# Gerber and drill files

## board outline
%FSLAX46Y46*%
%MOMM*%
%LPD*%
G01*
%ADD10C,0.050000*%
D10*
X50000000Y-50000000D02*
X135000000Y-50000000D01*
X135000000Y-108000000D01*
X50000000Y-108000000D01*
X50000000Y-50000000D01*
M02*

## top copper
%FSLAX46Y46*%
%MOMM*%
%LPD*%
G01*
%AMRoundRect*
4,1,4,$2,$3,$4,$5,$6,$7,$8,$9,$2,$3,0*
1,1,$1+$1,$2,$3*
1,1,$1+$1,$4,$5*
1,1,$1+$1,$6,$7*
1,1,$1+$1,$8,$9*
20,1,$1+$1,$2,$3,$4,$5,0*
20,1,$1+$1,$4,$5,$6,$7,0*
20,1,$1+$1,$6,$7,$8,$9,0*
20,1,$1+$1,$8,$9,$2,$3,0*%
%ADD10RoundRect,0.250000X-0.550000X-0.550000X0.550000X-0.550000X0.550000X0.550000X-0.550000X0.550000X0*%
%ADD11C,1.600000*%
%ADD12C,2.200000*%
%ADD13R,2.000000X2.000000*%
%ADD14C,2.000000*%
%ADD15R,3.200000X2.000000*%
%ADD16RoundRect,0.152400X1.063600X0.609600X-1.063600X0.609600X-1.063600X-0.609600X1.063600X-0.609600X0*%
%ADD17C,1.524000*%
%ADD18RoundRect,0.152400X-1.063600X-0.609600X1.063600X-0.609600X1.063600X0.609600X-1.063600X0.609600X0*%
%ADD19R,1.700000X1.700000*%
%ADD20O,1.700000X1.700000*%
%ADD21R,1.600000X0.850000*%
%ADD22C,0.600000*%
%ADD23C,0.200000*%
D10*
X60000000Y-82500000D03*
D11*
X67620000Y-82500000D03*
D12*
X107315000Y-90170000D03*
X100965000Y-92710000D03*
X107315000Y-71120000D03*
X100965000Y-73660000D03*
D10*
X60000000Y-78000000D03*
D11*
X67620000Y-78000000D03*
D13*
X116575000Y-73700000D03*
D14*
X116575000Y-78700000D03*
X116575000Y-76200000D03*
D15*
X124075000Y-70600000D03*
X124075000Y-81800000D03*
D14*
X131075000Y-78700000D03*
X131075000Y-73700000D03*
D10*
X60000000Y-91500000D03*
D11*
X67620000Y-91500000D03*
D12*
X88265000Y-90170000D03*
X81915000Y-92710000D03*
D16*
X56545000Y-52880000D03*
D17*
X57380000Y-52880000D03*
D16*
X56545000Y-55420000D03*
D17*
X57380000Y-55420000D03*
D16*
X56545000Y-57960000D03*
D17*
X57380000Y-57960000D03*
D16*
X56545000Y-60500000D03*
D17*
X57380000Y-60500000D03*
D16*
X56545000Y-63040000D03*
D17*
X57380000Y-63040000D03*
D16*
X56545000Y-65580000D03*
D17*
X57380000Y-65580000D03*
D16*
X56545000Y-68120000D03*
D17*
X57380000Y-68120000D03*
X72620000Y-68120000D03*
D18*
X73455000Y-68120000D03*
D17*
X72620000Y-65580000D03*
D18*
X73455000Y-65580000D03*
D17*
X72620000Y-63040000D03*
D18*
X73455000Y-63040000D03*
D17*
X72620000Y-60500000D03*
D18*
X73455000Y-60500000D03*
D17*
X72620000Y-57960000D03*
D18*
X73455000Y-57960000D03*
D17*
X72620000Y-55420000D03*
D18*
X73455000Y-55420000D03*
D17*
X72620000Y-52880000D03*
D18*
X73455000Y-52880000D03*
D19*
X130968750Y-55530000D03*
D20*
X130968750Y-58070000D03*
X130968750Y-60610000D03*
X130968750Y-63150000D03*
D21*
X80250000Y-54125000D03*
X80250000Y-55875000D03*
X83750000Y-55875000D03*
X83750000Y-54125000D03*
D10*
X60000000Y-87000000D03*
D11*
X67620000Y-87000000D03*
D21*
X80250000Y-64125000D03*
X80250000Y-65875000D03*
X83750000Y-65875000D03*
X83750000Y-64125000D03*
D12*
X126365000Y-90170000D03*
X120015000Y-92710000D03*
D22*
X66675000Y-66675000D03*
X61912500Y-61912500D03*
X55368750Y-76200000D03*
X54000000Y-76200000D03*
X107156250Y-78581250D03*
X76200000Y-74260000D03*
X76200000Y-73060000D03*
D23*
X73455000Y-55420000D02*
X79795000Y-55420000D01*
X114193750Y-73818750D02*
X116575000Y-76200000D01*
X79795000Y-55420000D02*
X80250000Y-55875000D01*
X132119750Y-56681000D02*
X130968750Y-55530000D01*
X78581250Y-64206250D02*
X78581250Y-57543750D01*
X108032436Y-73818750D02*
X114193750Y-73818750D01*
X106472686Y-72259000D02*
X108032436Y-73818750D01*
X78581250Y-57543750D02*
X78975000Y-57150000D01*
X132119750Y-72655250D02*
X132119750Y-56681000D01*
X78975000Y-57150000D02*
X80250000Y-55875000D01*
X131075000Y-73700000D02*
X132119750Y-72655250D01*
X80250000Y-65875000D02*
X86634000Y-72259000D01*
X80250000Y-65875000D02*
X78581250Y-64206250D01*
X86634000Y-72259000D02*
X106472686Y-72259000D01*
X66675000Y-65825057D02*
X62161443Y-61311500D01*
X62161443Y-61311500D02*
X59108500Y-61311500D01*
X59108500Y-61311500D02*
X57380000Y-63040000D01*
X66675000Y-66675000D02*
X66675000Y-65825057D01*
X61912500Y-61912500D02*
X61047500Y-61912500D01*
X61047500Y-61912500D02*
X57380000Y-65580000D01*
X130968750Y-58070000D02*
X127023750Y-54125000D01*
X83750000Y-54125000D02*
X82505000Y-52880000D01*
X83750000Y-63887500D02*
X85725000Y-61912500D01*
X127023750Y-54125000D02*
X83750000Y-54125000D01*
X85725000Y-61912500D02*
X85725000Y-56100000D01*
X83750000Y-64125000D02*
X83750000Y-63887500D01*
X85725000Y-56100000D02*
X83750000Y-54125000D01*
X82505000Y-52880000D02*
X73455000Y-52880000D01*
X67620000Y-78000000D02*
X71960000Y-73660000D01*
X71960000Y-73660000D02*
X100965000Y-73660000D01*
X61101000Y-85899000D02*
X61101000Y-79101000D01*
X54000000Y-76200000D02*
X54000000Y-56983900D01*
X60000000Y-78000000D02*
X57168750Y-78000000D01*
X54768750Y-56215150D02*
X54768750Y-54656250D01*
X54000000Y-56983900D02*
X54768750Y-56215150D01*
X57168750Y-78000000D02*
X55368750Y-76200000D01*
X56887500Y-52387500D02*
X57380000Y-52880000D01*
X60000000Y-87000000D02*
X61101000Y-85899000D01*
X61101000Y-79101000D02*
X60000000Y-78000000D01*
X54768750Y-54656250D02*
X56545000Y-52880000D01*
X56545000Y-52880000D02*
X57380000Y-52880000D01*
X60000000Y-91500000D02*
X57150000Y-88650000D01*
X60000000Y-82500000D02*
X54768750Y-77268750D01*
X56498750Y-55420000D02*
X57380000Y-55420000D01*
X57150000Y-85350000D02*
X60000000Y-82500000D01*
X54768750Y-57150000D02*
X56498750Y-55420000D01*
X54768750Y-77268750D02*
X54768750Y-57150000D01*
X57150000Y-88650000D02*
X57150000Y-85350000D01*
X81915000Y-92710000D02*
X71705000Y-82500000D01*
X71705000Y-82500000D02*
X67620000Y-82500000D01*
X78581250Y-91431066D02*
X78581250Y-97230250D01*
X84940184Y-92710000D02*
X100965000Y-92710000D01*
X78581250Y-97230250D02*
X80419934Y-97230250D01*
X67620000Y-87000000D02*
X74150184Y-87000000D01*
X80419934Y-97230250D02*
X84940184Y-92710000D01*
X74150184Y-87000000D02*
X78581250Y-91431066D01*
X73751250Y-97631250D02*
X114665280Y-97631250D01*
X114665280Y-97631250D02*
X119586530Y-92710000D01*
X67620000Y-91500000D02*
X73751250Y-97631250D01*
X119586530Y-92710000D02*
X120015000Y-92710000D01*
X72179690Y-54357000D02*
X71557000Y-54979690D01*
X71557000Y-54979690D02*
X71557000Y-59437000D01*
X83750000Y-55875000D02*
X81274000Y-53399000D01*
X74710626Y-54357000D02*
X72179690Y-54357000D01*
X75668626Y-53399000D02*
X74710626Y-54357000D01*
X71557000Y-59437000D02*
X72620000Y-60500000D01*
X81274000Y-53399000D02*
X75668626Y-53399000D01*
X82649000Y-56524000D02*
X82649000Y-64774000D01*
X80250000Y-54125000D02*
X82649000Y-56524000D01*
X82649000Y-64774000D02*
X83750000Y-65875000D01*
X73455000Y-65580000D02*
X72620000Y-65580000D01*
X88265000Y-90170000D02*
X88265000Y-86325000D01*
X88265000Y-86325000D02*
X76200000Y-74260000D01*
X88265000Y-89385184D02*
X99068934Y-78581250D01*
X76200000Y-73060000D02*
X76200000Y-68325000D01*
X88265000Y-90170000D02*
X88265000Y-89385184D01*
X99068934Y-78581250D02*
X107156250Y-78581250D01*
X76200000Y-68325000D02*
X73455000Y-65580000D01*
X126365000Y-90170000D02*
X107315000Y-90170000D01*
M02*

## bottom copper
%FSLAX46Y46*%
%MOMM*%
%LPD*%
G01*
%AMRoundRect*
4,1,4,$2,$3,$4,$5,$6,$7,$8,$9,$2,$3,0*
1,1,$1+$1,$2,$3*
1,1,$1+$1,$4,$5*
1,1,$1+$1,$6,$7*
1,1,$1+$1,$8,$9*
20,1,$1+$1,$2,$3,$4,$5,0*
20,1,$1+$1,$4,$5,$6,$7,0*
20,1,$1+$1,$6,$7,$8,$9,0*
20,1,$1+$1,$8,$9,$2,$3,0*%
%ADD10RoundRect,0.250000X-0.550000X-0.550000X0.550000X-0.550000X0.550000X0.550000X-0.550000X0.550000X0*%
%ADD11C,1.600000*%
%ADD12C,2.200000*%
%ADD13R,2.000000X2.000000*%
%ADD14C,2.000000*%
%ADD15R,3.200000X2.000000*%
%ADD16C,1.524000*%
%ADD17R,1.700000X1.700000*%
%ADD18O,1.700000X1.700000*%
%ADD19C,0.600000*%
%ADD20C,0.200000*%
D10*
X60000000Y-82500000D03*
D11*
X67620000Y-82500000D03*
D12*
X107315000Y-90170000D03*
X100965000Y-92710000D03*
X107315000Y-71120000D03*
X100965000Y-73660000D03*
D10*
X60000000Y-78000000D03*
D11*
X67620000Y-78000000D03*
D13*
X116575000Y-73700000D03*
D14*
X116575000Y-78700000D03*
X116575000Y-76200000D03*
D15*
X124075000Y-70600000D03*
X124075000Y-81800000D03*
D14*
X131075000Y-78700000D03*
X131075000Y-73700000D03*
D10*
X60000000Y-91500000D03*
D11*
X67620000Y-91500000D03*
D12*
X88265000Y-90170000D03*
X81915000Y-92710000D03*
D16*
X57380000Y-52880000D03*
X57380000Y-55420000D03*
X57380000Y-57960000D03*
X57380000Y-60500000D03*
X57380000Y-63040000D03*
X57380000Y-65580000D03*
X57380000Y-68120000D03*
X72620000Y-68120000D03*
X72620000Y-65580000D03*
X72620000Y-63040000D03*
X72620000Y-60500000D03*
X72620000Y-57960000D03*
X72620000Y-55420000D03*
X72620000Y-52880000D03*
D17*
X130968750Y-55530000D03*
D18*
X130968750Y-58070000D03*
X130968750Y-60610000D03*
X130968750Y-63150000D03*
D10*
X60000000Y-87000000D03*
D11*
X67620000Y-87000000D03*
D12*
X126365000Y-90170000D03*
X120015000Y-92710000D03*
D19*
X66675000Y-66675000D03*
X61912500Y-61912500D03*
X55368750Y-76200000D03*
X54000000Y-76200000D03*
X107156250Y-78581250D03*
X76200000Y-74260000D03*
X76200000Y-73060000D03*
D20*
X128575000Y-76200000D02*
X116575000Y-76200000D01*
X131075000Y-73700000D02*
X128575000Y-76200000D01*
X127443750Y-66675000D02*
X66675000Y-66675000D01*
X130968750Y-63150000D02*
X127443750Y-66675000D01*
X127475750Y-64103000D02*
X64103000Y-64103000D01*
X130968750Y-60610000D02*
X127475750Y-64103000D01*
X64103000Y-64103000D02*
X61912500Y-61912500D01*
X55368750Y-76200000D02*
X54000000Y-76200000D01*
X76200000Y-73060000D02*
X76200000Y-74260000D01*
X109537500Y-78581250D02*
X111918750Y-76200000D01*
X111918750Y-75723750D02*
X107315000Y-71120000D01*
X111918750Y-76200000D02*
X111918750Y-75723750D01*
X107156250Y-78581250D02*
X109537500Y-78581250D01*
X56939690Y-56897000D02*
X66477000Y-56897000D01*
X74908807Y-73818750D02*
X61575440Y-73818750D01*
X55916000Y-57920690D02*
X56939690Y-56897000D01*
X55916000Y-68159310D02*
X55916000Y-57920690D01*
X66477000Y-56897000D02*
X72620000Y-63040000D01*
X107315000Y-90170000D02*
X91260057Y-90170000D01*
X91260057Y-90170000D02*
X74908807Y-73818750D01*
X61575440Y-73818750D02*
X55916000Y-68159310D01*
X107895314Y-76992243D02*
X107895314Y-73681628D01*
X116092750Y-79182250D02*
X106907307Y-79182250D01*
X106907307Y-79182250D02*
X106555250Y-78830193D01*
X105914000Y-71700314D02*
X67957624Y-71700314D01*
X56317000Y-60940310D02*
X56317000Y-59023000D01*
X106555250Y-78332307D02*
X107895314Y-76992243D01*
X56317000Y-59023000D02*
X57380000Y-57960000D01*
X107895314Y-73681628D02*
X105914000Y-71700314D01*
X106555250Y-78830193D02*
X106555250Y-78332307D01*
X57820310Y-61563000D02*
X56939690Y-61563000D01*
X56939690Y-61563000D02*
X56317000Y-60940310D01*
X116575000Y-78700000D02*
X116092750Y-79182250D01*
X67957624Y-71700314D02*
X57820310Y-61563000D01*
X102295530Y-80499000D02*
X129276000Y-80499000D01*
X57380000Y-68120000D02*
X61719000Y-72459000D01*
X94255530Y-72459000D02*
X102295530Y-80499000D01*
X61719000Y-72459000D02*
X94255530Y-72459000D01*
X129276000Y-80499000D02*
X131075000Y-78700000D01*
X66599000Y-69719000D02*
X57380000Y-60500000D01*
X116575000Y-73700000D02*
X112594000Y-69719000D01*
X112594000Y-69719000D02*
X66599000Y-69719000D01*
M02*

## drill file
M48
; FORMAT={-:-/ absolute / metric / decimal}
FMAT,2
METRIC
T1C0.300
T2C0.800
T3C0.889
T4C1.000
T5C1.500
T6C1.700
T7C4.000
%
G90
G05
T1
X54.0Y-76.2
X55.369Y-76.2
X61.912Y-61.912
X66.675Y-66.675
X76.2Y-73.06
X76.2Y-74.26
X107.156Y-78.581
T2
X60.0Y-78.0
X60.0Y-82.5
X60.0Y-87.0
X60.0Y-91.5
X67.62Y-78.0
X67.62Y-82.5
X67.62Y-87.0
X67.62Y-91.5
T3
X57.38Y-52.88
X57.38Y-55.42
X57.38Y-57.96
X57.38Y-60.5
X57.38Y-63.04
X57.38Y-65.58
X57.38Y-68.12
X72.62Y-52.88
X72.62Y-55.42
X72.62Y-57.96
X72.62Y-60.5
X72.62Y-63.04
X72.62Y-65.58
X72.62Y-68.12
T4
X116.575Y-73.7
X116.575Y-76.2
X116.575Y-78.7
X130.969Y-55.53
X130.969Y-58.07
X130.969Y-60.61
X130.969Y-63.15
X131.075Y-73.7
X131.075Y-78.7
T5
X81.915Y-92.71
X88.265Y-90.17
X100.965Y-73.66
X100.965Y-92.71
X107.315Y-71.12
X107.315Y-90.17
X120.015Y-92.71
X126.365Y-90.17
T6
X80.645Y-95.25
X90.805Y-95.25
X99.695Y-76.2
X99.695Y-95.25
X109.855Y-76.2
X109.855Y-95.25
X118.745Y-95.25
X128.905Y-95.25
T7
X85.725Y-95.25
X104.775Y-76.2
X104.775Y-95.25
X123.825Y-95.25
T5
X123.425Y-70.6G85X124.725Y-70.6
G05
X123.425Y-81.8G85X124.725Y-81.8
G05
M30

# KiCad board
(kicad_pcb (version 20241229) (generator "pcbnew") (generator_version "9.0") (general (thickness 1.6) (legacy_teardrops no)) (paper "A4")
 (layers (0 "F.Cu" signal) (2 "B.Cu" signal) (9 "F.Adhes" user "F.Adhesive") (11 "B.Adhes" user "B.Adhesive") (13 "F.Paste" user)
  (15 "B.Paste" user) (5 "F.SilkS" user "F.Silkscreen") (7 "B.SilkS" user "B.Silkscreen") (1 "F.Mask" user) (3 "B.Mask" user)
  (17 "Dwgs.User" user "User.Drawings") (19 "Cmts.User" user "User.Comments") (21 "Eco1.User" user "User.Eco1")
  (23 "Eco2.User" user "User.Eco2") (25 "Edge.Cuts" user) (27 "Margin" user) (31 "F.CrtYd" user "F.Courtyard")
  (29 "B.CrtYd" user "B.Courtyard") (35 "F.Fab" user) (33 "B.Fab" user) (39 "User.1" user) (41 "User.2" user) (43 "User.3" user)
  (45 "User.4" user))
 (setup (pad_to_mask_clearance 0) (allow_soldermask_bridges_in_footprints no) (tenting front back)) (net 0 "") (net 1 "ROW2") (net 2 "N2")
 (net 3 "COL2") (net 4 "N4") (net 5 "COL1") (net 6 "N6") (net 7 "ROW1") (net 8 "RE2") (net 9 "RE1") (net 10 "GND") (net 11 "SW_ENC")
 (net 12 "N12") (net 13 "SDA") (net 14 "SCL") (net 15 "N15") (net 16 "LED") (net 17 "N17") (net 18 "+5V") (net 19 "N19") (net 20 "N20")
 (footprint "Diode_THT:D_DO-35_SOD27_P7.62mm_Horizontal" (layer "F.Cu") (at 60 82.5)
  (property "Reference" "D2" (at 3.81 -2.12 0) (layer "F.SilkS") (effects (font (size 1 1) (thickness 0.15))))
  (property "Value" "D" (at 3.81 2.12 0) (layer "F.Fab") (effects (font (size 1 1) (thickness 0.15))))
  (pad "1" thru_hole roundrect (at 0 0) (size 1.6 1.6) (drill 0.8) (layers "*.Cu" "*.Mask") (remove_unused_layers no)
   (roundrect_rratio 0.15625) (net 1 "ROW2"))
  (pad "2" thru_hole circle (at 7.62 0) (size 1.6 1.6) (drill 0.8) (layers "*.Cu" "*.Mask") (remove_unused_layers no) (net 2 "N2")))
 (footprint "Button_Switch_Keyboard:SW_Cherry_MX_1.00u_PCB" (layer "F.Cu") (at 107.315 90.17)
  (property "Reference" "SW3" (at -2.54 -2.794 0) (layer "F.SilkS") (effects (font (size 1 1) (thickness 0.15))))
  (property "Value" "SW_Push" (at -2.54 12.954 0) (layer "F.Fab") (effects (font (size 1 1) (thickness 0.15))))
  (pad "" np_thru_hole circle (at -7.62 5.08) (size 1.7 1.7) (drill 1.7) (layers "*.Cu" "*.Mask"))
  (pad "" np_thru_hole circle (at -2.54 5.08) (size 4 4) (drill 4) (layers "*.Cu" "*.Mask"))
  (pad "" np_thru_hole circle (at 2.54 5.08) (size 1.7 1.7) (drill 1.7) (layers "*.Cu" "*.Mask"))
  (pad "1" thru_hole circle (at 0 0) (size 2.2 2.2) (drill 1.5) (layers "*.Cu" "*.Mask") (remove_unused_layers no) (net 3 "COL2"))
  (pad "2" thru_hole circle (at -6.35 2.54) (size 2.2 2.2) (drill 1.5) (layers "*.Cu" "*.Mask") (remove_unused_layers no) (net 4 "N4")))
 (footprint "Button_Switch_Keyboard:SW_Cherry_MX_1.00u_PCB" (layer "F.Cu") (at 107.315 71.12)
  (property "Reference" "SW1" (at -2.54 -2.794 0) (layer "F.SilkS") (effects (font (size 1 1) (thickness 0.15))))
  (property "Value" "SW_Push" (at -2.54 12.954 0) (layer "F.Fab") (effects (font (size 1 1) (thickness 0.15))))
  (pad "" np_thru_hole circle (at -7.62 5.08) (size 1.7 1.7) (drill 1.7) (layers "*.Cu" "*.Mask"))
  (pad "" np_thru_hole circle (at -2.54 5.08) (size 4 4) (drill 4) (layers "*.Cu" "*.Mask"))
  (pad "" np_thru_hole circle (at 2.54 5.08) (size 1.7 1.7) (drill 1.7) (layers "*.Cu" "*.Mask"))
  (pad "1" thru_hole circle (at 0 0) (size 2.2 2.2) (drill 1.5) (layers "*.Cu" "*.Mask") (remove_unused_layers no) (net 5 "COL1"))
  (pad "2" thru_hole circle (at -6.35 2.54) (size 2.2 2.2) (drill 1.5) (layers "*.Cu" "*.Mask") (remove_unused_layers no) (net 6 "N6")))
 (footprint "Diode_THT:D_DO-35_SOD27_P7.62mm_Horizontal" (layer "F.Cu") (at 60 78)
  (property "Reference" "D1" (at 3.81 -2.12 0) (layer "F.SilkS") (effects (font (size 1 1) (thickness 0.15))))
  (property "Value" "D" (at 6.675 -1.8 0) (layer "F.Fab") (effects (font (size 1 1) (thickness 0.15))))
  (pad "1" thru_hole roundrect (at 0 0) (size 1.6 1.6) (drill 0.8) (layers "*.Cu" "*.Mask") (remove_unused_layers no)
   (roundrect_rratio 0.15625) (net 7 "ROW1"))
  (pad "2" thru_hole circle (at 7.62 0) (size 1.6 1.6) (drill 0.8) (layers "*.Cu" "*.Mask") (remove_unused_layers no) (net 6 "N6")))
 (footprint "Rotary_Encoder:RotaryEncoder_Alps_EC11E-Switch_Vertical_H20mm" (layer "F.Cu") (at 116.575 73.7)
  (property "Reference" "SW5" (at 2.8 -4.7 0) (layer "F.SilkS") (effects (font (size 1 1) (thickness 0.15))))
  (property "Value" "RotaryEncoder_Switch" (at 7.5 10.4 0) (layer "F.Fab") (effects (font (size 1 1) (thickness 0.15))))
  (pad "A" thru_hole rect (at 0 0) (size 2 2) (drill 1) (layers "*.Cu" "*.Mask") (remove_unused_layers no) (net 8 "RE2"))
  (pad "B" thru_hole circle (at 0 5) (size 2 2) (drill 1) (layers "*.Cu" "*.Mask") (remove_unused_layers no) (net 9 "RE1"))
  (pad "C" thru_hole circle (at 0 2.5) (size 2 2) (drill 1) (layers "*.Cu" "*.Mask") (remove_unused_layers no) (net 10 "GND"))
  (pad "MP" thru_hole rect (at 7.5 -3.1) (size 3.2 2) (drill oval 2.8 1.5) (layers "*.Cu" "*.Mask") (remove_unused_layers no))
  (pad "MP" thru_hole rect (at 7.5 8.1) (size 3.2 2) (drill oval 2.8 1.5) (layers "*.Cu" "*.Mask") (remove_unused_layers no))
  (pad "S1" thru_hole circle (at 14.5 5) (size 2 2) (drill 1) (layers "*.Cu" "*.Mask") (remove_unused_layers no) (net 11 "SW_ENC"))
  (pad "S2" thru_hole circle (at 14.5 0) (size 2 2) (drill 1) (layers "*.Cu" "*.Mask") (remove_unused_layers no) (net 10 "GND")))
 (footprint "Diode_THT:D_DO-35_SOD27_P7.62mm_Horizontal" (layer "F.Cu") (at 60 91.5)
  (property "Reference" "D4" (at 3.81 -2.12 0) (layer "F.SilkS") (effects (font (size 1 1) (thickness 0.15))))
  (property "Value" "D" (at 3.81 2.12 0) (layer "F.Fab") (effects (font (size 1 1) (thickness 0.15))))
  (pad "1" thru_hole roundrect (at 0 0) (size 1.6 1.6) (drill 0.8) (layers "*.Cu" "*.Mask") (remove_unused_layers no)
   (roundrect_rratio 0.15625) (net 1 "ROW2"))
  (pad "2" thru_hole circle (at 7.62 0) (size 1.6 1.6) (drill 0.8) (layers "*.Cu" "*.Mask") (remove_unused_layers no) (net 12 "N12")))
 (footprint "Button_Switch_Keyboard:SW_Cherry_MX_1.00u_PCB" (layer "F.Cu") (at 88.265 90.17)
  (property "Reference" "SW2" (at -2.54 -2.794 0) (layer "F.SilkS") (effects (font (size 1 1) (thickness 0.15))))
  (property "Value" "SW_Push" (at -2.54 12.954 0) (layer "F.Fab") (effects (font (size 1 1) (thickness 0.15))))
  (pad "" np_thru_hole circle (at -7.62 5.08) (size 1.7 1.7) (drill 1.7) (layers "*.Cu" "*.Mask"))
  (pad "" np_thru_hole circle (at -2.54 5.08) (size 4 4) (drill 4) (layers "*.Cu" "*.Mask"))
  (pad "" np_thru_hole circle (at 2.54 5.08) (size 1.7 1.7) (drill 1.7) (layers "*.Cu" "*.Mask"))
  (pad "1" thru_hole circle (at 0 0) (size 2.2 2.2) (drill 1.5) (layers "*.Cu" "*.Mask") (remove_unused_layers no) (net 5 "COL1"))
  (pad "2" thru_hole circle (at -6.35 2.54) (size 2.2 2.2) (drill 1.5) (layers "*.Cu" "*.Mask") (remove_unused_layers no) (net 2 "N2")))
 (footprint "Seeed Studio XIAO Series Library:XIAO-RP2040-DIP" (layer "F.Cu") (at 65 60.5)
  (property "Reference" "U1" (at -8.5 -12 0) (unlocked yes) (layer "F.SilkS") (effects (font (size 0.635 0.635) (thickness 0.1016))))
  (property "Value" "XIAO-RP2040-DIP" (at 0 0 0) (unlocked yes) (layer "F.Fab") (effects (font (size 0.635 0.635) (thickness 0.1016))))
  (pad "1" smd roundrect (at -8.455 -7.62 180) (size 2.432 1.524) (layers "F.Cu" "F.Mask") (roundrect_rratio 0.1) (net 7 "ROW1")
   (thermal_bridge_angle 45))
  (pad "1" thru_hole circle (at -7.62 -7.62 180) (size 1.524 1.524) (drill 0.889) (layers "*.Cu" "*.Mask") (remove_unused_layers no)
   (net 7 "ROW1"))
  (pad "2" smd roundrect (at -8.455 -5.08 180) (size 2.432 1.524) (layers "F.Cu" "F.Mask") (roundrect_rratio 0.1) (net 1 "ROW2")
   (thermal_bridge_angle 45))
  (pad "2" thru_hole circle (at -7.62 -5.08 180) (size 1.524 1.524) (drill 0.889) (layers "*.Cu" "*.Mask") (remove_unused_layers no)
   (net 1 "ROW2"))
  (pad "3" smd roundrect (at -8.455 -2.54 180) (size 2.432 1.524) (layers "F.Cu" "F.Mask") (roundrect_rratio 0.1) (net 9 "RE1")
   (thermal_bridge_angle 45))
  (pad "3" thru_hole circle (at -7.62 -2.54 180) (size 1.524 1.524) (drill 0.889) (layers "*.Cu" "*.Mask") (remove_unused_layers no)
   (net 9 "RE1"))
  (pad "4" smd roundrect (at -8.455 0 180) (size 2.432 1.524) (layers "F.Cu" "F.Mask") (roundrect_rratio 0.1) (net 8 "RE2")
   (thermal_bridge_angle 45))
  (pad "4" thru_hole circle (at -7.62 0 180) (size 1.524 1.524) (drill 0.889) (layers "*.Cu" "*.Mask") (remove_unused_layers no)
   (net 8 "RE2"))
  (pad "5" smd roundrect (at -8.455 2.54 180) (size 2.432 1.524) (layers "F.Cu" "F.Mask") (roundrect_rratio 0.1) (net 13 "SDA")
   (thermal_bridge_angle 45))
  (pad "5" thru_hole circle (at -7.62 2.54 180) (size 1.524 1.524) (drill 0.889) (layers "*.Cu" "*.Mask") (remove_unused_layers no)
   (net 13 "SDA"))
  (pad "6" smd roundrect (at -8.455 5.08 180) (size 2.432 1.524) (layers "F.Cu" "F.Mask") (roundrect_rratio 0.1) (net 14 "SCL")
   (thermal_bridge_angle 45))
  (pad "6" thru_hole circle (at -7.62 5.08 180) (size 1.524 1.524) (drill 0.889) (layers "*.Cu" "*.Mask") (remove_unused_layers no)
   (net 14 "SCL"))
  (pad "7" smd roundrect (at -8.455 7.62 180) (size 2.432 1.524) (layers "F.Cu" "F.Mask") (roundrect_rratio 0.1) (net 11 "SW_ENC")
   (thermal_bridge_angle 45))
  (pad "7" thru_hole circle (at -7.62 7.62 180) (size 1.524 1.524) (drill 0.889) (layers "*.Cu" "*.Mask") (remove_unused_layers no)
   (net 11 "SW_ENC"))
  (pad "8" thru_hole circle (at 7.62 7.62) (size 1.524 1.524) (drill 0.889) (layers "*.Cu" "*.Mask") (remove_unused_layers no)
   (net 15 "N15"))
  (pad "8" smd roundrect (at 8.455 7.62) (size 2.432 1.524) (layers "F.Cu" "F.Mask") (roundrect_rratio 0.1) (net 15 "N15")
   (thermal_bridge_angle 45))
  (pad "9" thru_hole circle (at 7.62 5.08) (size 1.524 1.524) (drill 0.889) (layers "*.Cu" "*.Mask") (remove_unused_layers no)
   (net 5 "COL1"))
  (pad "9" smd roundrect (at 8.455 5.08) (size 2.432 1.524) (layers "F.Cu" "F.Mask") (roundrect_rratio 0.1) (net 5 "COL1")
   (thermal_bridge_angle 45))
  (pad "10" thru_hole circle (at 7.62 2.54) (size 1.524 1.524) (drill 0.889) (layers "*.Cu" "*.Mask") (remove_unused_layers no)
   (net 3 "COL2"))
  (pad "10" smd roundrect (at 8.455 2.54) (size 2.432 1.524) (layers "F.Cu" "F.Mask") (roundrect_rratio 0.1) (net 3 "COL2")
   (thermal_bridge_angle 45))
  (pad "11" thru_hole circle (at 7.62 0) (size 1.524 1.524) (drill 0.889) (layers "*.Cu" "*.Mask") (remove_unused_layers no) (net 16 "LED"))
  (pad "11" smd roundrect (at 8.455 0) (size 2.432 1.524) (layers "F.Cu" "F.Mask") (roundrect_rratio 0.1) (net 16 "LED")
   (thermal_bridge_angle 45))
  (pad "12" thru_hole circle (at 7.62 -2.54) (size 1.524 1.524) (drill 0.889) (layers "*.Cu" "*.Mask") (remove_unused_layers no)
   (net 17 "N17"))
  (pad "12" smd roundrect (at 8.455 -2.54) (size 2.432 1.524) (layers "F.Cu" "F.Mask") (roundrect_rratio 0.1) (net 17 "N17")
   (thermal_bridge_angle 45))
  (pad "13" thru_hole circle (at 7.62 -5.08) (size 1.524 1.524) (drill 0.889) (layers "*.Cu" "*.Mask") (remove_unused_layers no)
   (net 10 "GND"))
  (pad "13" smd roundrect (at 8.455 -5.08) (size 2.432 1.524) (layers "F.Cu" "F.Mask") (roundrect_rratio 0.1) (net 10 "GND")
   (thermal_bridge_angle 45))
  (pad "14" thru_hole circle (at 7.62 -7.62) (size 1.524 1.524) (drill 0.889) (layers "*.Cu" "*.Mask") (remove_unused_layers no)
   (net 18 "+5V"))
  (pad "14" smd roundrect (at 8.455 -7.62) (size 2.432 1.524) (layers "F.Cu" "F.Mask") (roundrect_rratio 0.1) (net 18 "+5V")
   (thermal_bridge_angle 45)))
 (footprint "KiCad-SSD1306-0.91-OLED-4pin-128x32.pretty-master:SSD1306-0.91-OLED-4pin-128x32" (layer "F.Cu") (at 94.46875 53.34)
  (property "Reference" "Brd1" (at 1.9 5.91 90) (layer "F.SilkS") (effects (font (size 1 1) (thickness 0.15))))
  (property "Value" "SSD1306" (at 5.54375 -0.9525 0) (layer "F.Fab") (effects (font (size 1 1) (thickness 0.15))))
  (pad "1" thru_hole rect (at 36.5 2.19) (size 1.7 1.7) (drill 1) (layers "*.Cu" "*.Mask") (remove_unused_layers no) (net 10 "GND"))
  (pad "2" thru_hole oval (at 36.5 4.73) (size 1.7 1.7) (drill 1) (layers "*.Cu" "*.Mask") (remove_unused_layers no) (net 18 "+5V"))
  (pad "3" thru_hole oval (at 36.5 7.27) (size 1.7 1.7) (drill 1) (layers "*.Cu" "*.Mask") (remove_unused_layers no) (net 14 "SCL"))
  (pad "4" thru_hole oval (at 36.5 9.81) (size 1.7 1.7) (drill 1) (layers "*.Cu" "*.Mask") (remove_unused_layers no) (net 13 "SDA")))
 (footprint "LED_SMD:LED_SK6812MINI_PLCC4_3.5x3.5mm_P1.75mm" (layer "F.Cu") (at 82 55)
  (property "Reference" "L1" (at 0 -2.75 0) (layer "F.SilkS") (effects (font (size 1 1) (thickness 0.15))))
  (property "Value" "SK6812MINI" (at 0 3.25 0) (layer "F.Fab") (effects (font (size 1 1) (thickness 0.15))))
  (pad "1" smd rect (at -1.75 -0.875) (size 1.6 0.85) (layers "F.Cu" "F.Mask" "F.Paste") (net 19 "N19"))
  (pad "2" smd rect (at -1.75 0.875) (size 1.6 0.85) (layers "F.Cu" "F.Mask" "F.Paste") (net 10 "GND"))
  (pad "3" smd rect (at 1.75 0.875) (size 1.6 0.85) (layers "F.Cu" "F.Mask" "F.Paste") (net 16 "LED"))
  (pad "4" smd rect (at 1.75 -0.875) (size 1.6 0.85) (layers "F.Cu" "F.Mask" "F.Paste") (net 18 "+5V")))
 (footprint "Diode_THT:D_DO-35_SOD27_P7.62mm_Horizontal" (layer "F.Cu") (at 60 87)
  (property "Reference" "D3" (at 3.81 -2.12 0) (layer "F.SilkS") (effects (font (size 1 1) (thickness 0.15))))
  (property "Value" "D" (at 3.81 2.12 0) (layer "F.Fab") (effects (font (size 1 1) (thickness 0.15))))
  (pad "1" thru_hole roundrect (at 0 0) (size 1.6 1.6) (drill 0.8) (layers "*.Cu" "*.Mask") (remove_unused_layers no)
   (roundrect_rratio 0.15625) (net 7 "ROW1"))
  (pad "2" thru_hole circle (at 7.62 0) (size 1.6 1.6) (drill 0.8) (layers "*.Cu" "*.Mask") (remove_unused_layers no) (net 4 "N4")))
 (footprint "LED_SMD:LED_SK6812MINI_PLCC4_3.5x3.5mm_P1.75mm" (layer "F.Cu") (at 82 65)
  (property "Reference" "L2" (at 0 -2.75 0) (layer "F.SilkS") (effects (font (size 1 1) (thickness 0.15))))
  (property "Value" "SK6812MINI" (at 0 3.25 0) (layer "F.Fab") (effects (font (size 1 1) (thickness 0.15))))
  (pad "1" smd rect (at -1.75 -0.875) (size 1.6 0.85) (layers "F.Cu" "F.Mask" "F.Paste") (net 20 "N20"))
  (pad "2" smd rect (at -1.75 0.875) (size 1.6 0.85) (layers "F.Cu" "F.Mask" "F.Paste") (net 10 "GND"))
  (pad "3" smd rect (at 1.75 0.875) (size 1.6 0.85) (layers "F.Cu" "F.Mask" "F.Paste") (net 19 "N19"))
  (pad "4" smd rect (at 1.75 -0.875) (size 1.6 0.85) (layers "F.Cu" "F.Mask" "F.Paste") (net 18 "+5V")))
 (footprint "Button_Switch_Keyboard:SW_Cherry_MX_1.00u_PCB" (layer "F.Cu") (at 126.365 90.17)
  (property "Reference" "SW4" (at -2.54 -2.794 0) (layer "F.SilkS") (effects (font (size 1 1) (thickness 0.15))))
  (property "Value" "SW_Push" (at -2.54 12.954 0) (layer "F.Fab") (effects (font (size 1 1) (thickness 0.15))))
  (pad "" np_thru_hole circle (at -7.62 5.08) (size 1.7 1.7) (drill 1.7) (layers "*.Cu" "*.Mask"))
  (pad "" np_thru_hole circle (at -2.54 5.08) (size 4 4) (drill 4) (layers "*.Cu" "*.Mask"))
  (pad "" np_thru_hole circle (at 2.54 5.08) (size 1.7 1.7) (drill 1.7) (layers "*.Cu" "*.Mask"))
  (pad "1" thru_hole circle (at 0 0) (size 2.2 2.2) (drill 1.5) (layers "*.Cu" "*.Mask") (remove_unused_layers no) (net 3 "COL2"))
  (pad "2" thru_hole circle (at -6.35 2.54) (size 2.2 2.2) (drill 1.5) (layers "*.Cu" "*.Mask") (remove_unused_layers no) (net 12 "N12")))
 (gr_rect (start 50 50) (end 135 108) (stroke (width 0.05) (type solid)) (fill no) (layer "Edge.Cuts"))
 (segment (start 73.455 55.42) (end 79.795 55.42) (width 0.2) (layer "F.Cu") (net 10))
 (segment (start 114.19375 73.81875) (end 116.575 76.2) (width 0.2) (layer "F.Cu") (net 10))
 (segment (start 79.795 55.42) (end 80.25 55.875) (width 0.2) (layer "F.Cu") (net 10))
 (segment (start 132.11975 56.681) (end 130.96875 55.53) (width 0.2) (layer "F.Cu") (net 10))
 (segment (start 78.58125 64.20625) (end 78.58125 57.54375) (width 0.2) (layer "F.Cu") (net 10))
 (segment (start 108.032436 73.81875) (end 114.19375 73.81875) (width 0.2) (layer "F.Cu") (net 10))
 (segment (start 106.472686 72.259) (end 108.032436 73.81875) (width 0.2) (layer "F.Cu") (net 10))
 (segment (start 78.58125 57.54375) (end 78.975 57.15) (width 0.2) (layer "F.Cu") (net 10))
 (segment (start 132.11975 72.65525) (end 132.11975 56.681) (width 0.2) (layer "F.Cu") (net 10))
 (segment (start 78.975 57.15) (end 80.25 55.875) (width 0.2) (layer "F.Cu") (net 10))
 (segment (start 131.075 73.7) (end 132.11975 72.65525) (width 0.2) (layer "F.Cu") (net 10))
 (segment (start 80.25 65.875) (end 86.634 72.259) (width 0.2) (layer "F.Cu") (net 10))
 (segment (start 80.25 65.875) (end 78.58125 64.20625) (width 0.2) (layer "F.Cu") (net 10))
 (segment (start 86.634 72.259) (end 106.472686 72.259) (width 0.2) (layer "F.Cu") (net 10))
 (segment (start 128.575 76.2) (end 116.575 76.2) (width 0.2) (layer "B.Cu") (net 10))
 (segment (start 131.075 73.7) (end 128.575 76.2) (width 0.2) (layer "B.Cu") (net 10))
 (segment (start 66.675 65.825057) (end 62.161443 61.3115) (width 0.2) (layer "F.Cu") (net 13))
 (segment (start 62.161443 61.3115) (end 59.1085 61.3115) (width 0.2) (layer "F.Cu") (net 13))
 (segment (start 59.1085 61.3115) (end 57.38 63.04) (width 0.2) (layer "F.Cu") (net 13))
 (segment (start 66.675 66.675) (end 66.675 65.825057) (width 0.2) (layer "F.Cu") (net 13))
 (via (at 66.675 66.675) (size 0.6) (drill 0.3) (layers "F.Cu" "B.Cu") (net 13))
 (segment (start 127.44375 66.675) (end 66.675 66.675) (width 0.2) (layer "B.Cu") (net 13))
 (segment (start 130.96875 63.15) (end 127.44375 66.675) (width 0.2) (layer "B.Cu") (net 13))
 (segment (start 61.9125 61.9125) (end 61.0475 61.9125) (width 0.2) (layer "F.Cu") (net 14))
 (segment (start 61.0475 61.9125) (end 57.38 65.58) (width 0.2) (layer "F.Cu") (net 14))
 (via (at 61.9125 61.9125) (size 0.6) (drill 0.3) (layers "F.Cu" "B.Cu") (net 14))
 (segment (start 127.47575 64.103) (end 64.103 64.103) (width 0.2) (layer "B.Cu") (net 14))
 (segment (start 130.96875 60.61) (end 127.47575 64.103) (width 0.2) (layer "B.Cu") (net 14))
 (segment (start 64.103 64.103) (end 61.9125 61.9125) (width 0.2) (layer "B.Cu") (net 14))
 (segment (start 130.96875 58.07) (end 127.02375 54.125) (width 0.2) (layer "F.Cu") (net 18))
 (segment (start 83.75 54.125) (end 82.505 52.88) (width 0.2) (layer "F.Cu") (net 18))
 (segment (start 83.75 63.8875) (end 85.725 61.9125) (width 0.2) (layer "F.Cu") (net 18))
 (segment (start 127.02375 54.125) (end 83.75 54.125) (width 0.2) (layer "F.Cu") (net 18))
 (segment (start 85.725 61.9125) (end 85.725 56.1) (width 0.2) (layer "F.Cu") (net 18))
 (segment (start 83.75 64.125) (end 83.75 63.8875) (width 0.2) (layer "F.Cu") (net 18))
 (segment (start 85.725 56.1) (end 83.75 54.125) (width 0.2) (layer "F.Cu") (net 18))
 (segment (start 82.505 52.88) (end 73.455 52.88) (width 0.2) (layer "F.Cu") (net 18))
 (segment (start 67.62 78) (end 71.96 73.66) (width 0.2) (layer "F.Cu") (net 6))
 (segment (start 71.96 73.66) (end 100.965 73.66) (width 0.2) (layer "F.Cu") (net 6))
 (segment (start 61.101 85.899) (end 61.101 79.101) (width 0.2) (layer "F.Cu") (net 7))
 (segment (start 54 76.2) (end 54 56.9839) (width 0.2) (layer "F.Cu") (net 7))
 (segment (start 60 78) (end 57.16875 78) (width 0.2) (layer "F.Cu") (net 7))
 (segment (start 54.76875 56.21515) (end 54.76875 54.65625) (width 0.2) (layer "F.Cu") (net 7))
 (segment (start 54 56.9839) (end 54.76875 56.21515) (width 0.2) (layer "F.Cu") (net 7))
 (segment (start 57.16875 78) (end 55.36875 76.2) (width 0.2) (layer "F.Cu") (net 7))
 (segment (start 56.8875 52.3875) (end 57.38 52.88) (width 0.2) (layer "F.Cu") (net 7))
 (segment (start 60 87) (end 61.101 85.899) (width 0.2) (layer "F.Cu") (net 7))
 (segment (start 61.101 79.101) (end 60 78) (width 0.2) (layer "F.Cu") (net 7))
 (segment (start 54.76875 54.65625) (end 56.545 52.88) (width 0.2) (layer "F.Cu") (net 7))
 (segment (start 56.545 52.88) (end 57.38 52.88) (width 0.2) (layer "F.Cu") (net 7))
 (via (at 55.36875 76.2) (size 0.6) (drill 0.3) (layers "F.Cu" "B.Cu") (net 7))
 (via (at 54 76.2) (size 0.6) (drill 0.3) (layers "F.Cu" "B.Cu") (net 7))
 (segment (start 55.36875 76.2) (end 54 76.2) (width 0.2) (layer "B.Cu") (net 7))
 (segment (start 60 91.5) (end 57.15 88.65) (width 0.2) (layer "F.Cu") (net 1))
 (segment (start 60 82.5) (end 54.76875 77.26875) (width 0.2) (layer "F.Cu") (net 1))
 (segment (start 56.49875 55.42) (end 57.38 55.42) (width 0.2) (layer "F.Cu") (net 1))
 (segment (start 57.15 85.35) (end 60 82.5) (width 0.2) (layer "F.Cu") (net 1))
 (segment (start 54.76875 57.15) (end 56.49875 55.42) (width 0.2) (layer "F.Cu") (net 1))
 (segment (start 54.76875 77.26875) (end 54.76875 57.15) (width 0.2) (layer "F.Cu") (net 1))
 (segment (start 57.15 88.65) (end 57.15 85.35) (width 0.2) (layer "F.Cu") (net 1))
 (segment (start 81.915 92.71) (end 71.705 82.5) (width 0.2) (layer "F.Cu") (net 2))
 (segment (start 71.705 82.5) (end 67.62 82.5) (width 0.2) (layer "F.Cu") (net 2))
 (segment (start 78.58125 91.431066) (end 78.58125 97.23025) (width 0.2) (layer "F.Cu") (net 4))
 (segment (start 84.940184 92.71) (end 100.965 92.71) (width 0.2) (layer "F.Cu") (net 4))
 (segment (start 78.58125 97.23025) (end 80.419934 97.23025) (width 0.2) (layer "F.Cu") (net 4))
 (segment (start 67.62 87) (end 74.150184 87) (width 0.2) (layer "F.Cu") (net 4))
 (segment (start 80.419934 97.23025) (end 84.940184 92.71) (width 0.2) (layer "F.Cu") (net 4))
 (segment (start 74.150184 87) (end 78.58125 91.431066) (width 0.2) (layer "F.Cu") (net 4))
 (segment (start 73.75125 97.63125) (end 114.66528 97.63125) (width 0.2) (layer "F.Cu") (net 12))
 (segment (start 114.66528 97.63125) (end 119.58653 92.71) (width 0.2) (layer "F.Cu") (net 12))
 (segment (start 67.62 91.5) (end 73.75125 97.63125) (width 0.2) (layer "F.Cu") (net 12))
 (segment (start 119.58653 92.71) (end 120.015 92.71) (width 0.2) (layer "F.Cu") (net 12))
 (segment (start 72.17969 54.357) (end 71.557 54.97969) (width 0.2) (layer "F.Cu") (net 16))
 (segment (start 71.557 54.97969) (end 71.557 59.437) (width 0.2) (layer "F.Cu") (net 16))
 (segment (start 83.75 55.875) (end 81.274 53.399) (width 0.2) (layer "F.Cu") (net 16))
 (segment (start 74.710626 54.357) (end 72.17969 54.357) (width 0.2) (layer "F.Cu") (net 16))
 (segment (start 75.668626 53.399) (end 74.710626 54.357) (width 0.2) (layer "F.Cu") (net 16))
 (segment (start 71.557 59.437) (end 72.62 60.5) (width 0.2) (layer "F.Cu") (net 16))
 (segment (start 81.274 53.399) (end 75.668626 53.399) (width 0.2) (layer "F.Cu") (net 16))
 (segment (start 82.649 56.524) (end 82.649 64.774) (width 0.2) (layer "F.Cu") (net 19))
 (segment (start 80.25 54.125) (end 82.649 56.524) (width 0.2) (layer "F.Cu") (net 19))
 (segment (start 82.649 64.774) (end 83.75 65.875) (width 0.2) (layer "F.Cu") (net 19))
 (segment (start 73.455 65.58) (end 72.62 65.58) (width 0.2) (layer "F.Cu") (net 5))
 (segment (start 88.265 90.17) (end 88.265 86.325) (width 0.2) (layer "F.Cu") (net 5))
 (segment (start 88.265 86.325) (end 76.2 74.26) (width 0.2) (layer "F.Cu") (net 5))
 (segment (start 88.265 89.385184) (end 99.068934 78.58125) (width 0.2) (layer "F.Cu") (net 5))
 (segment (start 76.2 73.06) (end 76.2 68.325) (width 0.2) (layer "F.Cu") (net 5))
 (segment (start 88.265 90.17) (end 88.265 89.385184) (width 0.2) (layer "F.Cu") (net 5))
 (segment (start 99.068934 78.58125) (end 107.15625 78.58125) (width 0.2) (layer "F.Cu") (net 5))
 (segment (start 76.2 68.325) (end 73.455 65.58) (width 0.2) (layer "F.Cu") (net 5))
 (via (at 107.15625 78.58125) (size 0.6) (drill 0.3) (layers "F.Cu" "B.Cu") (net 5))
 (via (at 76.2 74.26) (size 0.6) (drill 0.3) (layers "F.Cu" "B.Cu") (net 5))
 (via (at 76.2 73.06) (size 0.6) (drill 0.3) (layers "F.Cu" "B.Cu") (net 5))
 (segment (start 76.2 73.06) (end 76.2 74.26) (width 0.2) (layer "B.Cu") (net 5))
 (segment (start 109.5375 78.58125) (end 111.91875 76.2) (width 0.2) (layer "B.Cu") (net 5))
 (segment (start 111.91875 75.72375) (end 107.315 71.12) (width 0.2) (layer "B.Cu") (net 5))
 (segment (start 111.91875 76.2) (end 111.91875 75.72375) (width 0.2) (layer "B.Cu") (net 5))
 (segment (start 107.15625 78.58125) (end 109.5375 78.58125) (width 0.2) (layer "B.Cu") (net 5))
 (segment (start 126.365 90.17) (end 107.315 90.17) (width 0.2) (layer "F.Cu") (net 3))
 (segment (start 56.93969 56.897) (end 66.477 56.897) (width 0.2) (layer "B.Cu") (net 3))
 (segment (start 74.908807 73.81875) (end 61.57544 73.81875) (width 0.2) (layer "B.Cu") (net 3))
 (segment (start 55.916 57.92069) (end 56.93969 56.897) (width 0.2) (layer "B.Cu") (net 3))
 (segment (start 55.916 68.15931) (end 55.916 57.92069) (width 0.2) (layer "B.Cu") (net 3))
 (segment (start 66.477 56.897) (end 72.62 63.04) (width 0.2) (layer "B.Cu") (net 3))
 (segment (start 107.315 90.17) (end 91.260057 90.17) (width 0.2) (layer "B.Cu") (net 3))
 (segment (start 91.260057 90.17) (end 74.908807 73.81875) (width 0.2) (layer "B.Cu") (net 3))
 (segment (start 61.57544 73.81875) (end 55.916 68.15931) (width 0.2) (layer "B.Cu") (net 3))
 (segment (start 107.895314 76.992243) (end 107.895314 73.681628) (width 0.2) (layer "B.Cu") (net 9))
 (segment (start 116.09275 79.18225) (end 106.907307 79.18225) (width 0.2) (layer "B.Cu") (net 9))
 (segment (start 106.907307 79.18225) (end 106.55525 78.830193) (width 0.2) (layer "B.Cu") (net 9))
 (segment (start 105.914 71.700314) (end 67.957624 71.700314) (width 0.2) (layer "B.Cu") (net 9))
 (segment (start 56.317 60.94031) (end 56.317 59.023) (width 0.2) (layer "B.Cu") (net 9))
 (segment (start 106.55525 78.332307) (end 107.895314 76.992243) (width 0.2) (layer "B.Cu") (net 9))
 (segment (start 56.317 59.023) (end 57.38 57.96) (width 0.2) (layer "B.Cu") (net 9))
 (segment (start 107.895314 73.681628) (end 105.914 71.700314) (width 0.2) (layer "B.Cu") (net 9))
 (segment (start 106.55525 78.830193) (end 106.55525 78.332307) (width 0.2) (layer "B.Cu") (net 9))
 (segment (start 57.82031 61.563) (end 56.93969 61.563) (width 0.2) (layer "B.Cu") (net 9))
 (segment (start 56.93969 61.563) (end 56.317 60.94031) (width 0.2) (layer "B.Cu") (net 9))
 (segment (start 116.575 78.7) (end 116.09275 79.18225) (width 0.2) (layer "B.Cu") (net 9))
 (segment (start 67.957624 71.700314) (end 57.82031 61.563) (width 0.2) (layer "B.Cu") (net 9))
 (segment (start 102.29553 80.499) (end 129.276 80.499) (width 0.2) (layer "B.Cu") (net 11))
 (segment (start 57.38 68.12) (end 61.719 72.459) (width 0.2) (layer "B.Cu") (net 11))
 (segment (start 94.25553 72.459) (end 102.29553 80.499) (width 0.2) (layer "B.Cu") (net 11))
 (segment (start 61.719 72.459) (end 94.25553 72.459) (width 0.2) (layer "B.Cu") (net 11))
 (segment (start 129.276 80.499) (end 131.075 78.7) (width 0.2) (layer "B.Cu") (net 11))
 (segment (start 66.599 69.719) (end 57.38 60.5) (width 0.2) (layer "B.Cu") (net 8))
 (segment (start 116.575 73.7) (end 112.594 69.719) (width 0.2) (layer "B.Cu") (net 8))
 (segment (start 112.594 69.719) (end 66.599 69.719) (width 0.2) (layer "B.Cu") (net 8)))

